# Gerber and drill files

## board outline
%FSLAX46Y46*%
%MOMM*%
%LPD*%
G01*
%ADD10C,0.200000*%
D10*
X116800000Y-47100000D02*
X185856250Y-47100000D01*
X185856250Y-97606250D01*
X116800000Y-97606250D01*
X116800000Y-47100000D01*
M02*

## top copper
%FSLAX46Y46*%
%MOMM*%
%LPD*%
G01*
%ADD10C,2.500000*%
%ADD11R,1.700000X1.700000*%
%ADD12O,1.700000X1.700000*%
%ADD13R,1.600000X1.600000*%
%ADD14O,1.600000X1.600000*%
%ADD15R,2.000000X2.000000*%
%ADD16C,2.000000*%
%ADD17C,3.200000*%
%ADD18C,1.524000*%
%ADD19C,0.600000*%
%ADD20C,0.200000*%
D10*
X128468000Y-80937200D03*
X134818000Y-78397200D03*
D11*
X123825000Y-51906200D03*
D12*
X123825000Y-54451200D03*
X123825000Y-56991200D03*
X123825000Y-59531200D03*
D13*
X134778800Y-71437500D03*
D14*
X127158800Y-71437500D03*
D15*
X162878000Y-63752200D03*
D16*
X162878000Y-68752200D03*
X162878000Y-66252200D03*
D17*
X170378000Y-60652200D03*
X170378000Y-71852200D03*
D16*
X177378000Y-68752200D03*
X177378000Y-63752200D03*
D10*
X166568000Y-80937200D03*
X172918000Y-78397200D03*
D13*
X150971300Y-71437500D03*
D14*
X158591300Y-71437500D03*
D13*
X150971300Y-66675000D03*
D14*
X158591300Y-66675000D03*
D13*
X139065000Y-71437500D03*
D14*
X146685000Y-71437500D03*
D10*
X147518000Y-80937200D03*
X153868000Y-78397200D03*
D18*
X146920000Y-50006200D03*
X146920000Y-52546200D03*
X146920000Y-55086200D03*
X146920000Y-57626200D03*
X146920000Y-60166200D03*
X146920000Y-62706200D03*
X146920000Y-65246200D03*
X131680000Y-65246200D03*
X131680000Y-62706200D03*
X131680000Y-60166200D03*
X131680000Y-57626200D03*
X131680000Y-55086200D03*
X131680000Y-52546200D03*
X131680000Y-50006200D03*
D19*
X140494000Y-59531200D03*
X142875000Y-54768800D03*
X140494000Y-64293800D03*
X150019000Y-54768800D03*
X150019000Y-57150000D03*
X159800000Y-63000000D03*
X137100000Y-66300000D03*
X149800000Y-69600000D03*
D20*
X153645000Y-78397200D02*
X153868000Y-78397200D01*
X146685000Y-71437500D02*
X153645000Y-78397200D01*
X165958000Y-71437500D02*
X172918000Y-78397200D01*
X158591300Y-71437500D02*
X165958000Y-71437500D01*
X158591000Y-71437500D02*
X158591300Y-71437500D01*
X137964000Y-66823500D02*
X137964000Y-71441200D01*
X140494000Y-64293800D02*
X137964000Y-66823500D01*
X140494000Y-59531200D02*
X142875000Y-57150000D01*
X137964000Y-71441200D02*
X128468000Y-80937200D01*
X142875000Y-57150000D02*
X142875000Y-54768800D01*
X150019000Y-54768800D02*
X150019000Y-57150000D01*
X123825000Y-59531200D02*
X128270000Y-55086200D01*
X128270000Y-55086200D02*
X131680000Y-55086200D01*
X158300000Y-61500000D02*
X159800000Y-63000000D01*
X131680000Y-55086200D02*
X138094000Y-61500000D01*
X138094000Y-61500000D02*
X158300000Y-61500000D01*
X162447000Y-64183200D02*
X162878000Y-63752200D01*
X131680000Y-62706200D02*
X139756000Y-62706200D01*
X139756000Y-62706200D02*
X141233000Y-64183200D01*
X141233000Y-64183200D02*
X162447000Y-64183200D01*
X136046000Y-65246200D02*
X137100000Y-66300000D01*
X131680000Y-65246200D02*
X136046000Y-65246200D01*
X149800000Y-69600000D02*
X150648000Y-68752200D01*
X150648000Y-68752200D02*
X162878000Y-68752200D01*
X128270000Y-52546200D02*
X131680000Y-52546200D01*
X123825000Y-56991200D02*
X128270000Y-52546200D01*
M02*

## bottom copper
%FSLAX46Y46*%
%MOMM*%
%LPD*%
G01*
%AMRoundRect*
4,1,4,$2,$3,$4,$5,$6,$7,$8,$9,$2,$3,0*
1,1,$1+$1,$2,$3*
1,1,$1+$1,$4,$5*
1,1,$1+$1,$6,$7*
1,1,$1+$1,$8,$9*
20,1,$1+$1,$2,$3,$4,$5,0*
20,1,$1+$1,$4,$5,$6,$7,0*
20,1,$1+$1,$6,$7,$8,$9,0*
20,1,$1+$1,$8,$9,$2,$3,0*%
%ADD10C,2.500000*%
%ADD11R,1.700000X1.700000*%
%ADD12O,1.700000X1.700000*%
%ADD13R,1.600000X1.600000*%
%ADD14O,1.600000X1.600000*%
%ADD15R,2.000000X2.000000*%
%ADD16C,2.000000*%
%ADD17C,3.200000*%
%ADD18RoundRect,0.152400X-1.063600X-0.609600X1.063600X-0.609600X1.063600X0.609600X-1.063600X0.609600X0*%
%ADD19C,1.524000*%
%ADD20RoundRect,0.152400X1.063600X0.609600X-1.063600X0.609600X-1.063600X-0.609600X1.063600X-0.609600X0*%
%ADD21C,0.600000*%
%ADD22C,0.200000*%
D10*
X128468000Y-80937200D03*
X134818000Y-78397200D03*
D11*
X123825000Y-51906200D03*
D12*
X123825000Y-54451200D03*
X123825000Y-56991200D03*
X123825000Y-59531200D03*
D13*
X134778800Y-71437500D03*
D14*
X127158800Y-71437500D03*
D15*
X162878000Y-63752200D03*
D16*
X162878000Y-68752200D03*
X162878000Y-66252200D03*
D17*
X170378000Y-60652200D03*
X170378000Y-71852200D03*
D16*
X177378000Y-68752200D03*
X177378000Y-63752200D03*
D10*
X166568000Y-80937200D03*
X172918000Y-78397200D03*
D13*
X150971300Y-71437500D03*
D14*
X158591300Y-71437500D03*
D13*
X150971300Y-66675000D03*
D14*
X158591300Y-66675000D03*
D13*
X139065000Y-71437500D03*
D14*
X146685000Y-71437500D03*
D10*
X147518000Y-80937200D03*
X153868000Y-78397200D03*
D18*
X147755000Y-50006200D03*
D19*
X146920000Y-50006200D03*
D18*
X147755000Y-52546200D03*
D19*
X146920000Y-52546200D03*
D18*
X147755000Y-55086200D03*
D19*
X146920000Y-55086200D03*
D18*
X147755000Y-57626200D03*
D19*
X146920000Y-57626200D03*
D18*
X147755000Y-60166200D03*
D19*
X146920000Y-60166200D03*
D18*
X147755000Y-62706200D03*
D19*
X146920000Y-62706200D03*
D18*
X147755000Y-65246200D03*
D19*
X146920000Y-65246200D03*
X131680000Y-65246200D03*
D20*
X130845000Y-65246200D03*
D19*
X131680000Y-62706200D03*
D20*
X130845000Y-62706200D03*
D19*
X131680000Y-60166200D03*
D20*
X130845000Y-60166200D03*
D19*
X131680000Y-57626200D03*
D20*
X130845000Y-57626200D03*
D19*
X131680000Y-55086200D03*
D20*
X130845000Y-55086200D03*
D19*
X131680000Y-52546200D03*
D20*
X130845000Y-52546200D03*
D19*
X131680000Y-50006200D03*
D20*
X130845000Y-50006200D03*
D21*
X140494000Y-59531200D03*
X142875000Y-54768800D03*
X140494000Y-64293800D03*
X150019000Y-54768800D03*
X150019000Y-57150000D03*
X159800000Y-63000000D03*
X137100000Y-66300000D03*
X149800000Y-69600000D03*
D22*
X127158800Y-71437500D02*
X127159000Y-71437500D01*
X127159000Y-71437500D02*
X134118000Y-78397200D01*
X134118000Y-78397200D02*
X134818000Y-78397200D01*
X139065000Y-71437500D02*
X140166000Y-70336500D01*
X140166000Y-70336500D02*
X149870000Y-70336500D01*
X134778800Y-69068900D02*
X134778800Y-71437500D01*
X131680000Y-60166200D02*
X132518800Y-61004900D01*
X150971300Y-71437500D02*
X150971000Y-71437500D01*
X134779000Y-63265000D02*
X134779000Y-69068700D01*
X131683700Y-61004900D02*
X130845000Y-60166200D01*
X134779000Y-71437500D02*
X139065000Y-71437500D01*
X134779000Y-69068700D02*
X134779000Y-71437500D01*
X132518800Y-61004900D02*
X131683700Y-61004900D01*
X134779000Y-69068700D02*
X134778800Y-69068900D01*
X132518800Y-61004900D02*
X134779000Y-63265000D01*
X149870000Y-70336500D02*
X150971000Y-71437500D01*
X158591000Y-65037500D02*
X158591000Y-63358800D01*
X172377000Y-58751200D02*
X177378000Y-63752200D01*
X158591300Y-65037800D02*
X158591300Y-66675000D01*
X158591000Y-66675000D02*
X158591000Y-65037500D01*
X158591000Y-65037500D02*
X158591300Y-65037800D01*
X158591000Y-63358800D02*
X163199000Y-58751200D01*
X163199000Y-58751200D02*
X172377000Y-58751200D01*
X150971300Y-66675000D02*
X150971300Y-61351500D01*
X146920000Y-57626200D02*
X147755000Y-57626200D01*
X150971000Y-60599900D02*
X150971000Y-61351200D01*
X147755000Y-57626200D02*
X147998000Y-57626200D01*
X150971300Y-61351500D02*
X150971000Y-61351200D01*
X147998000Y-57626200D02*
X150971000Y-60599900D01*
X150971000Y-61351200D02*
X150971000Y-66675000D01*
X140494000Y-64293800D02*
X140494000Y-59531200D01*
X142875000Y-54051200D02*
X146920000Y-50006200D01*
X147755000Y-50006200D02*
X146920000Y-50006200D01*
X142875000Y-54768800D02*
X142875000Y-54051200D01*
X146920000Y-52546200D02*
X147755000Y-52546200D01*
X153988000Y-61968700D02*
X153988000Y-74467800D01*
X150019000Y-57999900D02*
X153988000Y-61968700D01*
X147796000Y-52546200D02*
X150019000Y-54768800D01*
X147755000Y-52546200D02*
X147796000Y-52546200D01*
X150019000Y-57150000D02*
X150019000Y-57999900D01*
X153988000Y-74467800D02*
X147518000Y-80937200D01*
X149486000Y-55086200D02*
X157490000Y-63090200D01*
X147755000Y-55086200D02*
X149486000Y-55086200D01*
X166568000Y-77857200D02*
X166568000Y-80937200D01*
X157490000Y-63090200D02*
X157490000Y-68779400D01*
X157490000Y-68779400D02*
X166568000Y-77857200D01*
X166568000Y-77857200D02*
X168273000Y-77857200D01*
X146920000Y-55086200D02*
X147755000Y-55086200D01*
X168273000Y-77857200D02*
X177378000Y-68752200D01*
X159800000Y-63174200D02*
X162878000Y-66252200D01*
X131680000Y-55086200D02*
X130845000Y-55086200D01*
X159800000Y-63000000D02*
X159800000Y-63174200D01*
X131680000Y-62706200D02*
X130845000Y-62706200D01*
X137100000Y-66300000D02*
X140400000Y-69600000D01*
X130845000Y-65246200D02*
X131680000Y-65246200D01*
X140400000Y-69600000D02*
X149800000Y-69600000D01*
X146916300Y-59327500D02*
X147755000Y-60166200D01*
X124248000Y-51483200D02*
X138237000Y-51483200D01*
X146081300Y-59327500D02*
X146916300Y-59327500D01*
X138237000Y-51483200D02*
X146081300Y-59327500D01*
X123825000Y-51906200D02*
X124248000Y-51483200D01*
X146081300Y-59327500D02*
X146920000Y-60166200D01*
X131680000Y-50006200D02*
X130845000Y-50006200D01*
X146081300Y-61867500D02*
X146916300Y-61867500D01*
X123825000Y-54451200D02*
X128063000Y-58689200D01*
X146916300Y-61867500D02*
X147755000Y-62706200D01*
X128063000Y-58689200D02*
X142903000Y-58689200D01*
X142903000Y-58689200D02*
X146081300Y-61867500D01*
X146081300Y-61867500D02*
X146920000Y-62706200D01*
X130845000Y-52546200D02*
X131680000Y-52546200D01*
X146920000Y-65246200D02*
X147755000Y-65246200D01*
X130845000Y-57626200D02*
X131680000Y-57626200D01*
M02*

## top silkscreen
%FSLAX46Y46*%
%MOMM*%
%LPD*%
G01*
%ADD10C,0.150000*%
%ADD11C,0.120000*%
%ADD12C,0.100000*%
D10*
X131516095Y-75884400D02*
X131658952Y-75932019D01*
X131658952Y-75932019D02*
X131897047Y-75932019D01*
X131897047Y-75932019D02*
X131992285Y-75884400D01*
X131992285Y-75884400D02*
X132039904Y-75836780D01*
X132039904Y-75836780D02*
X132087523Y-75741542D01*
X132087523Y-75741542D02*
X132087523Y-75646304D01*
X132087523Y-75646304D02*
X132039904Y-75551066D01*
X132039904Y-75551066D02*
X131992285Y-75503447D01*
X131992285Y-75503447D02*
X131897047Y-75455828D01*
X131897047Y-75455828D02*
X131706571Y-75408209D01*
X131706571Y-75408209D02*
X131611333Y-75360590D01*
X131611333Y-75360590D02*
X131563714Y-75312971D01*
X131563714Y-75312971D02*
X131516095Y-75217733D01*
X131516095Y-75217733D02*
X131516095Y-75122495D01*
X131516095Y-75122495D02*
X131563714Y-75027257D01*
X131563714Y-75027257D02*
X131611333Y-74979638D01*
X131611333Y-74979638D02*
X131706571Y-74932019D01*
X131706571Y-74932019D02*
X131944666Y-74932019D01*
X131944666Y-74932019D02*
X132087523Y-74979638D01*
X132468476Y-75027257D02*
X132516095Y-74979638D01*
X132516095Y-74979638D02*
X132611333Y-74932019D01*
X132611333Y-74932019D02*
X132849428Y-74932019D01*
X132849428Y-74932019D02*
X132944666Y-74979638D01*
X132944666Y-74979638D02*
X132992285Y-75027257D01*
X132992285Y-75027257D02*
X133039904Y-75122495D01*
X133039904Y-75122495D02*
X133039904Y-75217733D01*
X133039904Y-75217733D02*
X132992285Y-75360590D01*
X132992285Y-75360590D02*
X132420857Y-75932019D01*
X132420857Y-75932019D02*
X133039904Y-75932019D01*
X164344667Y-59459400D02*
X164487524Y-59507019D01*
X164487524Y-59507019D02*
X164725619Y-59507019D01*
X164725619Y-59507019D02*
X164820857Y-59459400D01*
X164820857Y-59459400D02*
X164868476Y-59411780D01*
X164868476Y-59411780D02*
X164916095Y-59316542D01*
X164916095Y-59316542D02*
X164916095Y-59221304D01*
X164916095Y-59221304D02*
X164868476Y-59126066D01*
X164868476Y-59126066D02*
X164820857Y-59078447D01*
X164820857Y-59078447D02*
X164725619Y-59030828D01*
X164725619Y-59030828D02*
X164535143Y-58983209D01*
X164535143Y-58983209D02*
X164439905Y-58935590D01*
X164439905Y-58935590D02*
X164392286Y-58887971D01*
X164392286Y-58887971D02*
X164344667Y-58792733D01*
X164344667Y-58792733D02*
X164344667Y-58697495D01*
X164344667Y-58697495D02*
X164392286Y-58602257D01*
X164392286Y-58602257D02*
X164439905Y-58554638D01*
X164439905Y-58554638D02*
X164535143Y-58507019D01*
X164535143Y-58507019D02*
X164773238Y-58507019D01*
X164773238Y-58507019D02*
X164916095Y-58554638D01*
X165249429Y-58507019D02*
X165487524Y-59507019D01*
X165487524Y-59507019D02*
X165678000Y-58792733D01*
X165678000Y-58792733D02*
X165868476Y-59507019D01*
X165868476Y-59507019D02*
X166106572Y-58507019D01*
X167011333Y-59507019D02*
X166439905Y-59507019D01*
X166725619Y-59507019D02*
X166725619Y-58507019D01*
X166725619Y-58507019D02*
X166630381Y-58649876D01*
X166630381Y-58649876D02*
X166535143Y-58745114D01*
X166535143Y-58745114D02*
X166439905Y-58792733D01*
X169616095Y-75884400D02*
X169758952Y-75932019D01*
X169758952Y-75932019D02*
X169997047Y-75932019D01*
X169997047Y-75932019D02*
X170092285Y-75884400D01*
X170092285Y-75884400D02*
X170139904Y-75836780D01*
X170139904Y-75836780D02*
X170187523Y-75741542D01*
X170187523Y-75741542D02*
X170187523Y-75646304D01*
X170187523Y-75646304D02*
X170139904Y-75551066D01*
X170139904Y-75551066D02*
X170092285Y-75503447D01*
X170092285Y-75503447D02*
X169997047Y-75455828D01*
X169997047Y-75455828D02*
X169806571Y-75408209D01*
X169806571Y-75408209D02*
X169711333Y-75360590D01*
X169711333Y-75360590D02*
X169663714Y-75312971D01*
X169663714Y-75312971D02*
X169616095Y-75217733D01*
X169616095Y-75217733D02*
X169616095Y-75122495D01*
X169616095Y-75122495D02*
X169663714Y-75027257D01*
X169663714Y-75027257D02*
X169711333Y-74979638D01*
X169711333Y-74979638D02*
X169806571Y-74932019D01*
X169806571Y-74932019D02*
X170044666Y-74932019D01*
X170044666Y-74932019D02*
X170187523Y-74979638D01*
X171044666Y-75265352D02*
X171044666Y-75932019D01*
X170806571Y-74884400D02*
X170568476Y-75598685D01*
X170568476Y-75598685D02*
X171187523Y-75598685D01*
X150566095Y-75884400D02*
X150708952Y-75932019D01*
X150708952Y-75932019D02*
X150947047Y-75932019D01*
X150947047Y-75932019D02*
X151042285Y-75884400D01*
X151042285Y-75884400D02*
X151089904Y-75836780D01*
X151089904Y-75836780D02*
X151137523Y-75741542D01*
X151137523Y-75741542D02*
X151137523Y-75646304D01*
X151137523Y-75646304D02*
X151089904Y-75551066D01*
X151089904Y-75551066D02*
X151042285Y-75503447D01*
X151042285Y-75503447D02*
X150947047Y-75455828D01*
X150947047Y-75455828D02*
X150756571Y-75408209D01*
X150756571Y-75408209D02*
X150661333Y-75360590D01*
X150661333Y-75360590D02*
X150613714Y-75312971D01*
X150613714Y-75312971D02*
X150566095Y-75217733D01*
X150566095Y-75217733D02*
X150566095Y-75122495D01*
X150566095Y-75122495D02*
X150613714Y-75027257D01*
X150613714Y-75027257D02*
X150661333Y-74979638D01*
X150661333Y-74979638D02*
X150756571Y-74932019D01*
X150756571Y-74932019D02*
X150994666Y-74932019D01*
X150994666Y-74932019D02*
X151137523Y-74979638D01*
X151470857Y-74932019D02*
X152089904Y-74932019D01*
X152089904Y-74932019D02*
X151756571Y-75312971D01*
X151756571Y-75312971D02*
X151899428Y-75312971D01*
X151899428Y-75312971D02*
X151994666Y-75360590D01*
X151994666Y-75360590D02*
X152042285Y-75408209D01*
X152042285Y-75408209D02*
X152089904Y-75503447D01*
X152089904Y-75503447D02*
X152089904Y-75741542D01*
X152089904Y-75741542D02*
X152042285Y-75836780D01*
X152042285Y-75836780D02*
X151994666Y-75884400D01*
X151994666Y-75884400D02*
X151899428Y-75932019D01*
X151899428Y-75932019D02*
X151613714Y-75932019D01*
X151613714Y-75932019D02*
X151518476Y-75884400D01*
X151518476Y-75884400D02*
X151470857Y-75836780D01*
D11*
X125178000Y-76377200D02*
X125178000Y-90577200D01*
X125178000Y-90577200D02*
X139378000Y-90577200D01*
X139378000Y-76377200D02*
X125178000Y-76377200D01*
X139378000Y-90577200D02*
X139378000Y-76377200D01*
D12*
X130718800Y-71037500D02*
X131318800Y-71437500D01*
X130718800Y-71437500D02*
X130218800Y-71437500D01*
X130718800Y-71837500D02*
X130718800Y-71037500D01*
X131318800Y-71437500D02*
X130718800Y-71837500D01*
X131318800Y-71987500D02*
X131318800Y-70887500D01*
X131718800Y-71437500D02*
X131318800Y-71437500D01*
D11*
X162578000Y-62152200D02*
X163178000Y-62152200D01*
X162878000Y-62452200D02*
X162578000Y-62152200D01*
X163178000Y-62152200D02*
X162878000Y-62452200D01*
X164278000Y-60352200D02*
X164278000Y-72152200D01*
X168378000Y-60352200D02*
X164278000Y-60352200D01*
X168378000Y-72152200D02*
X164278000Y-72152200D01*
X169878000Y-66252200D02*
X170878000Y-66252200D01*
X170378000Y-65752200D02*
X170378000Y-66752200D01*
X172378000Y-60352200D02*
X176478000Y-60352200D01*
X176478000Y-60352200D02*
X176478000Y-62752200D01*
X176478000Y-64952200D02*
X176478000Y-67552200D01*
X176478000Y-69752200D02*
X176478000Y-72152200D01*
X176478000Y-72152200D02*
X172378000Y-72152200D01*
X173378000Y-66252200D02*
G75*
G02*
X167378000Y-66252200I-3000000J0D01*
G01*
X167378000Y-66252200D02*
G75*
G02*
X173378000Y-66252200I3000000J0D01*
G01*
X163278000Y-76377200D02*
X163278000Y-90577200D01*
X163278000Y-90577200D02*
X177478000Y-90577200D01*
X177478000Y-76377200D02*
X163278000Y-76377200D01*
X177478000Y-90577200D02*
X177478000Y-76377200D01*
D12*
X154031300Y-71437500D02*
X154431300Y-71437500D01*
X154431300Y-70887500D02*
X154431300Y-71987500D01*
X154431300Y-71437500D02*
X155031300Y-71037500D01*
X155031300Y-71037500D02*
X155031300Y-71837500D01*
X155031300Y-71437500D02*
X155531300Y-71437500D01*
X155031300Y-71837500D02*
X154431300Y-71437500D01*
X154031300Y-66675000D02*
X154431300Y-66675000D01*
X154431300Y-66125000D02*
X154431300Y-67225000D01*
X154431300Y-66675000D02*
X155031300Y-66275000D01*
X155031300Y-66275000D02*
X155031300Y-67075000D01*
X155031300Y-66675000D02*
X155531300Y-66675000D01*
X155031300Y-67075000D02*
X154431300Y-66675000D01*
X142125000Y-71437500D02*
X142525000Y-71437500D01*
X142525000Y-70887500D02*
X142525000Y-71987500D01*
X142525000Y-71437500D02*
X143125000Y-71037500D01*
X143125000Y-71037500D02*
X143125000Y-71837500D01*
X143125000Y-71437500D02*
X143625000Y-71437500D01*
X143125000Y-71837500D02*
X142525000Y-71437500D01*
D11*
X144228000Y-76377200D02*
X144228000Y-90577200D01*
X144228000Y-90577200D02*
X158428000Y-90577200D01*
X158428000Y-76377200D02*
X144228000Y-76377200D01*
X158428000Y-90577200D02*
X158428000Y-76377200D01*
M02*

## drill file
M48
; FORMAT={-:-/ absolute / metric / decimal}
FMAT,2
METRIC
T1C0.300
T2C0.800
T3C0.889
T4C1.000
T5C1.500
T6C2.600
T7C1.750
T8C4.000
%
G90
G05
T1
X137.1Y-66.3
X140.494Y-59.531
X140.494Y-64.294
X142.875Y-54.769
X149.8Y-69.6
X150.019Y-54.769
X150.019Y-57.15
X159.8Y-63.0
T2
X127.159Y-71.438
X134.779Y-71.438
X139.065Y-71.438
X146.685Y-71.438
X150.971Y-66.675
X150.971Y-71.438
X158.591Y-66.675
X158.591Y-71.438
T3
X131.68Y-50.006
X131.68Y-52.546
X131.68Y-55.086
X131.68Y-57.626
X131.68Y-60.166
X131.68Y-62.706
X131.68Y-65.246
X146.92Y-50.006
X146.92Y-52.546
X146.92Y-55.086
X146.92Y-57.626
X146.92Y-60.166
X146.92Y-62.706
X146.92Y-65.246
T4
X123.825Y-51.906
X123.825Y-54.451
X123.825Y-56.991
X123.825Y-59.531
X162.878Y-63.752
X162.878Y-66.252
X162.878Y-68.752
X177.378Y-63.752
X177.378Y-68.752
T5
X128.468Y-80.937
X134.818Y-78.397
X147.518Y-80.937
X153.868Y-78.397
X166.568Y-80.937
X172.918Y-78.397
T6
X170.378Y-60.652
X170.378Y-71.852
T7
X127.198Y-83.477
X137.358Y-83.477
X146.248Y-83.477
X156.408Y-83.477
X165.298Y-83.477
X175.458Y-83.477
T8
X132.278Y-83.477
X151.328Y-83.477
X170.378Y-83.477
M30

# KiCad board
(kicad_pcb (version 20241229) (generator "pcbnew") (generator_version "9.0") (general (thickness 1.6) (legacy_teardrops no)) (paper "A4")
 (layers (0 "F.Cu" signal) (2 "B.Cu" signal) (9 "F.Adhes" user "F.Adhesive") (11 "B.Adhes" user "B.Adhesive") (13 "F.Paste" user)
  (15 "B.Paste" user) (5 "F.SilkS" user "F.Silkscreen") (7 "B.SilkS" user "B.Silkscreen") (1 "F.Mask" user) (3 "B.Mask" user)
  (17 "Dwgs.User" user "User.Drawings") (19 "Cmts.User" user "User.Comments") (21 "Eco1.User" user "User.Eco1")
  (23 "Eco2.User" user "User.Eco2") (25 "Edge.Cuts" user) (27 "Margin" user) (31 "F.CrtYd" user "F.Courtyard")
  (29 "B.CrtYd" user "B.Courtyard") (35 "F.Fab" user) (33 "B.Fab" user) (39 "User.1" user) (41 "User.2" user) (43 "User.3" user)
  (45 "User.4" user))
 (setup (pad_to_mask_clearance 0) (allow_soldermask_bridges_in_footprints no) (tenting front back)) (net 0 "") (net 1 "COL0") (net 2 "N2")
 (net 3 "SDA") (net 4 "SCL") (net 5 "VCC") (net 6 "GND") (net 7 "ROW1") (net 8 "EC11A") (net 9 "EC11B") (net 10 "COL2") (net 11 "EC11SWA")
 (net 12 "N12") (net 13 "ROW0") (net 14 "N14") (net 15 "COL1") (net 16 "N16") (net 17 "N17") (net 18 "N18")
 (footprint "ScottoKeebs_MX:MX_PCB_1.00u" (layer "F.Cu") (at 132.278 83.4772)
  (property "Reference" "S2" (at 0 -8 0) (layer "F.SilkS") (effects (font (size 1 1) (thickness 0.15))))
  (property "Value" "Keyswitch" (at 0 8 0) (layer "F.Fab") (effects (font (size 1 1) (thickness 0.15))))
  (fp_line (start -7.1 -7.1) (end -7.1 7.1) (stroke (width 0.12) (type solid)) (layer "F.SilkS"))
  (fp_line (start -7.1 7.1) (end 7.1 7.1) (stroke (width 0.12) (type solid)) (layer "F.SilkS"))
  (fp_line (start 7.1 -7.1) (end -7.1 -7.1) (stroke (width 0.12) (type solid)) (layer "F.SilkS"))
  (fp_line (start 7.1 7.1) (end 7.1 -7.1) (stroke (width 0.12) (type solid)) (layer "F.SilkS"))
  (pad "" np_thru_hole circle (at -5.08 0) (size 1.75 1.75) (drill 1.75) (layers "*.Cu" "*.Mask"))
  (pad "" np_thru_hole circle (at 0 0) (size 4 4) (drill 4) (layers "*.Cu" "*.Mask"))
  (pad "" np_thru_hole circle (at 5.08 0) (size 1.75 1.75) (drill 1.75) (layers "*.Cu" "*.Mask"))
  (pad "1" thru_hole circle (at -3.81 -2.54) (size 2.5 2.5) (drill 1.5) (layers "*.Cu" "*.Mask") (remove_unused_layers no) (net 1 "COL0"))
  (pad "2" thru_hole circle (at 2.54 -5.08) (size 2.5 2.5) (drill 1.5) (layers "*.Cu" "*.Mask") (remove_unused_layers no) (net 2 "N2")))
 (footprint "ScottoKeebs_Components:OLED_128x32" (layer "F.Cu") (at 122.225 49.7312)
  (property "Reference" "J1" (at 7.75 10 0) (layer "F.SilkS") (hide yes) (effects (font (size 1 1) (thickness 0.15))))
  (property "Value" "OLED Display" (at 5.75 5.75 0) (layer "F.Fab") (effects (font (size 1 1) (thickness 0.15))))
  (pad "1" thru_hole rect (at 1.6 2.175 180) (size 1.7 1.7) (drill 1) (layers "*.Cu" "*.Mask") (remove_unused_layers no) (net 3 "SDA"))
  (pad "2" thru_hole oval (at 1.6 4.72 180) (size 1.7 1.7) (drill 1) (layers "*.Cu" "*.Mask") (remove_unused_layers no) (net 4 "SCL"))
  (pad "3" thru_hole oval (at 1.6 7.26 180) (size 1.7 1.7) (drill 1) (layers "*.Cu" "*.Mask") (remove_unused_layers no) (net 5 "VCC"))
  (pad "4" thru_hole oval (at 1.6 9.8 180) (size 1.7 1.7) (drill 1) (layers "*.Cu" "*.Mask") (remove_unused_layers no) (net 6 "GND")))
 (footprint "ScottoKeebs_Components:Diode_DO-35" (layer "F.Cu") (at 134.7788 71.4375 180)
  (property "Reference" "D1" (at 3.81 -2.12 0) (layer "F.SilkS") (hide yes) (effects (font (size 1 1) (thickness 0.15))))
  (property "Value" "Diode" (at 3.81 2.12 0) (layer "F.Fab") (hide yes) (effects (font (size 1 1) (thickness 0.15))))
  (fp_line (start 4.06 0.4) (end 3.46 0) (stroke (width 0.1) (type solid)) (layer "F.SilkS"))
  (fp_line (start 4.06 0) (end 4.56 0) (stroke (width 0.1) (type solid)) (layer "F.SilkS"))
  (fp_line (start 4.06 -0.4) (end 4.06 0.4) (stroke (width 0.1) (type solid)) (layer "F.SilkS"))
  (fp_line (start 3.46 0) (end 4.06 -0.4) (stroke (width 0.1) (type solid)) (layer "F.SilkS"))
  (fp_line (start 3.46 -0.55) (end 3.46 0.55) (stroke (width 0.1) (type solid)) (layer "F.SilkS"))
  (fp_line (start 3.06 0) (end 3.46 0) (stroke (width 0.1) (type solid)) (layer "F.SilkS"))
  (pad "1" thru_hole rect (at 0 0 180) (size 1.6 1.6) (drill 0.8) (layers "*.Cu" "*.Mask") (remove_unused_layers no) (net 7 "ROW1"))
  (pad "2" thru_hole oval (at 7.62 0 180) (size 1.6 1.6) (drill 0.8) (layers "*.Cu" "*.Mask") (remove_unused_layers no) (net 2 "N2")))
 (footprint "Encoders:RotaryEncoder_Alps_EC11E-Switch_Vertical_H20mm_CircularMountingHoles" (layer "F.Cu") (at 162.878 63.7522)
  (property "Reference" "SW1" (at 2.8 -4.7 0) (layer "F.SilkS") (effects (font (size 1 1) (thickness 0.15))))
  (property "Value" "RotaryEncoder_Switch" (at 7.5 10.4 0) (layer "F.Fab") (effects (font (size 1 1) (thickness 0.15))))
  (fp_line (start -0.3 -1.6) (end 0.3 -1.6) (stroke (width 0.12) (type solid)) (layer "F.SilkS"))
  (fp_line (start 0 -1.3) (end -0.3 -1.6) (stroke (width 0.12) (type solid)) (layer "F.SilkS"))
  (fp_line (start 0.3 -1.6) (end 0 -1.3) (stroke (width 0.12) (type solid)) (layer "F.SilkS"))
  (fp_line (start 1.4 -3.4) (end 1.4 8.4) (stroke (width 0.12) (type solid)) (layer "F.SilkS"))
  (fp_line (start 5.5 -3.4) (end 1.4 -3.4) (stroke (width 0.12) (type solid)) (layer "F.SilkS"))
  (fp_line (start 5.5 8.4) (end 1.4 8.4) (stroke (width 0.12) (type solid)) (layer "F.SilkS"))
  (fp_line (start 7 2.5) (end 8 2.5) (stroke (width 0.12) (type solid)) (layer "F.SilkS"))
  (fp_line (start 7.5 2) (end 7.5 3) (stroke (width 0.12) (type solid)) (layer "F.SilkS"))
  (fp_line (start 9.5 -3.4) (end 13.6 -3.4) (stroke (width 0.12) (type solid)) (layer "F.SilkS"))
  (fp_line (start 13.6 -3.4) (end 13.6 -1) (stroke (width 0.12) (type solid)) (layer "F.SilkS"))
  (fp_line (start 13.6 1.2) (end 13.6 3.8) (stroke (width 0.12) (type solid)) (layer "F.SilkS"))
  (fp_line (start 13.6 6) (end 13.6 8.4) (stroke (width 0.12) (type solid)) (layer "F.SilkS"))
  (fp_line (start 13.6 8.4) (end 9.5 8.4) (stroke (width 0.12) (type solid)) (layer "F.SilkS"))
  (fp_circle (center 7.5 2.5) (end 10.5 2.5) (stroke (width 0.12) (type solid)) (fill no) (layer "F.SilkS"))
  (pad "A" thru_hole rect (at 0 0) (size 2 2) (drill 1) (layers "*.Cu" "*.Mask") (remove_unused_layers no) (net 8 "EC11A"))
  (pad "B" thru_hole circle (at 0 5) (size 2 2) (drill 1) (layers "*.Cu" "*.Mask") (remove_unused_layers no) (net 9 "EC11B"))
  (pad "C" thru_hole circle (at 0 2.5) (size 2 2) (drill 1) (layers "*.Cu" "*.Mask") (remove_unused_layers no) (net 6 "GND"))
  (pad "MP" thru_hole circle (at 7.5 -3.1) (size 3.2 3.2) (drill 2.6) (layers "*.Cu" "*.Mask") (remove_unused_layers no))
  (pad "MP" thru_hole circle (at 7.5 8.1) (size 3.2 3.2) (drill 2.6) (layers "*.Cu" "*.Mask") (remove_unused_layers no))
  (pad "S1" thru_hole circle (at 14.5 5) (size 2 2) (drill 1) (layers "*.Cu" "*.Mask") (remove_unused_layers no) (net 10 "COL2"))
  (pad "S2" thru_hole circle (at 14.5 0) (size 2 2) (drill 1) (layers "*.Cu" "*.Mask") (remove_unused_layers no) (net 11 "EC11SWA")))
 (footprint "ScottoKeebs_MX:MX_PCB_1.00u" (layer "F.Cu") (at 170.378 83.4772)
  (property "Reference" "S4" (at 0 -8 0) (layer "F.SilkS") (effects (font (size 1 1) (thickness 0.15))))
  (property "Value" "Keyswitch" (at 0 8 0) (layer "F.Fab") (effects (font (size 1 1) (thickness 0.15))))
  (fp_line (start -7.1 -7.1) (end -7.1 7.1) (stroke (width 0.12) (type solid)) (layer "F.SilkS"))
  (fp_line (start -7.1 7.1) (end 7.1 7.1) (stroke (width 0.12) (type solid)) (layer "F.SilkS"))
  (fp_line (start 7.1 -7.1) (end -7.1 -7.1) (stroke (width 0.12) (type solid)) (layer "F.SilkS"))
  (fp_line (start 7.1 7.1) (end 7.1 -7.1) (stroke (width 0.12) (type solid)) (layer "F.SilkS"))
  (pad "" np_thru_hole circle (at -5.08 0) (size 1.75 1.75) (drill 1.75) (layers "*.Cu" "*.Mask"))
  (pad "" np_thru_hole circle (at 0 0) (size 4 4) (drill 4) (layers "*.Cu" "*.Mask"))
  (pad "" np_thru_hole circle (at 5.08 0) (size 1.75 1.75) (drill 1.75) (layers "*.Cu" "*.Mask"))
  (pad "1" thru_hole circle (at -3.81 -2.54) (size 2.5 2.5) (drill 1.5) (layers "*.Cu" "*.Mask") (remove_unused_layers no) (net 10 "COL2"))
  (pad "2" thru_hole circle (at 2.54 -5.08) (size 2.5 2.5) (drill 1.5) (layers "*.Cu" "*.Mask") (remove_unused_layers no) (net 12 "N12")))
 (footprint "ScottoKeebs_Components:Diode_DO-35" (layer "F.Cu") (at 150.9713 71.4375)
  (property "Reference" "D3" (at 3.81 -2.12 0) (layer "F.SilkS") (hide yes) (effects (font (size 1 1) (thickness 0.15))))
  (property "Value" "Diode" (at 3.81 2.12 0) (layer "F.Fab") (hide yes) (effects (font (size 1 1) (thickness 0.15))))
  (fp_line (start 3.06 0) (end 3.46 0) (stroke (width 0.1) (type solid)) (layer "F.SilkS"))
  (fp_line (start 3.46 -0.55) (end 3.46 0.55) (stroke (width 0.1) (type solid)) (layer "F.SilkS"))
  (fp_line (start 3.46 0) (end 4.06 -0.4) (stroke (width 0.1) (type solid)) (layer "F.SilkS"))
  (fp_line (start 4.06 -0.4) (end 4.06 0.4) (stroke (width 0.1) (type solid)) (layer "F.SilkS"))
  (fp_line (start 4.06 0) (end 4.56 0) (stroke (width 0.1) (type solid)) (layer "F.SilkS"))
  (fp_line (start 4.06 0.4) (end 3.46 0) (stroke (width 0.1) (type solid)) (layer "F.SilkS"))
  (pad "1" thru_hole rect (at 0 0) (size 1.6 1.6) (drill 0.8) (layers "*.Cu" "*.Mask") (remove_unused_layers no) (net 7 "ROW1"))
  (pad "2" thru_hole oval (at 7.62 0) (size 1.6 1.6) (drill 0.8) (layers "*.Cu" "*.Mask") (remove_unused_layers no) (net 12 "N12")))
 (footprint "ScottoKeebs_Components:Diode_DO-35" (layer "F.Cu") (at 150.9713 66.675)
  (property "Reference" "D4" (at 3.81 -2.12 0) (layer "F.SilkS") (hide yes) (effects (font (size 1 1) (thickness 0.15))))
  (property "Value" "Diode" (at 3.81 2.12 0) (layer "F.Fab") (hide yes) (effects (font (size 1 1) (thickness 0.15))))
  (fp_line (start 3.06 0) (end 3.46 0) (stroke (width 0.1) (type solid)) (layer "F.SilkS"))
  (fp_line (start 3.46 -0.55) (end 3.46 0.55) (stroke (width 0.1) (type solid)) (layer "F.SilkS"))
  (fp_line (start 3.46 0) (end 4.06 -0.4) (stroke (width 0.1) (type solid)) (layer "F.SilkS"))
  (fp_line (start 4.06 -0.4) (end 4.06 0.4) (stroke (width 0.1) (type solid)) (layer "F.SilkS"))
  (fp_line (start 4.06 0) (end 4.56 0) (stroke (width 0.1) (type solid)) (layer "F.SilkS"))
  (fp_line (start 4.06 0.4) (end 3.46 0) (stroke (width 0.1) (type solid)) (layer "F.SilkS"))
  (pad "1" thru_hole rect (at 0 0) (size 1.6 1.6) (drill 0.8) (layers "*.Cu" "*.Mask") (remove_unused_layers no) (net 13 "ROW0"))
  (pad "2" thru_hole oval (at 7.62 0) (size 1.6 1.6) (drill 0.8) (layers "*.Cu" "*.Mask") (remove_unused_layers no) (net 11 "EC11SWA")))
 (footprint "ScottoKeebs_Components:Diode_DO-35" (layer "F.Cu") (at 139.065 71.4375)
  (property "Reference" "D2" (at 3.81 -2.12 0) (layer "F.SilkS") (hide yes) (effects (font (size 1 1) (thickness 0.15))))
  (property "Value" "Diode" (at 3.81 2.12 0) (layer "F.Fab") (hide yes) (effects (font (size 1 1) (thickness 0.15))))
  (fp_line (start 3.06 0) (end 3.46 0) (stroke (width 0.1) (type solid)) (layer "F.SilkS"))
  (fp_line (start 3.46 -0.55) (end 3.46 0.55) (stroke (width 0.1) (type solid)) (layer "F.SilkS"))
  (fp_line (start 3.46 0) (end 4.06 -0.4) (stroke (width 0.1) (type solid)) (layer "F.SilkS"))
  (fp_line (start 4.06 -0.4) (end 4.06 0.4) (stroke (width 0.1) (type solid)) (layer "F.SilkS"))
  (fp_line (start 4.06 0) (end 4.56 0) (stroke (width 0.1) (type solid)) (layer "F.SilkS"))
  (fp_line (start 4.06 0.4) (end 3.46 0) (stroke (width 0.1) (type solid)) (layer "F.SilkS"))
  (pad "1" thru_hole rect (at 0 0) (size 1.6 1.6) (drill 0.8) (layers "*.Cu" "*.Mask") (remove_unused_layers no) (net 7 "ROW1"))
  (pad "2" thru_hole oval (at 7.62 0) (size 1.6 1.6) (drill 0.8) (layers "*.Cu" "*.Mask") (remove_unused_layers no) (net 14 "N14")))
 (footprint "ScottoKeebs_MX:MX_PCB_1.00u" (layer "F.Cu") (at 151.328 83.4772)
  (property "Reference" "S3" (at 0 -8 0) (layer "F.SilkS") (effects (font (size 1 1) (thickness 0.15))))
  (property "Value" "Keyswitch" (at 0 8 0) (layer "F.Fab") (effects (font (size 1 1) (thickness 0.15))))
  (fp_line (start -7.1 -7.1) (end -7.1 7.1) (stroke (width 0.12) (type solid)) (layer "F.SilkS"))
  (fp_line (start -7.1 7.1) (end 7.1 7.1) (stroke (width 0.12) (type solid)) (layer "F.SilkS"))
  (fp_line (start 7.1 -7.1) (end -7.1 -7.1) (stroke (width 0.12) (type solid)) (layer "F.SilkS"))
  (fp_line (start 7.1 7.1) (end 7.1 -7.1) (stroke (width 0.12) (type solid)) (layer "F.SilkS"))
  (pad "" np_thru_hole circle (at -5.08 0) (size 1.75 1.75) (drill 1.75) (layers "*.Cu" "*.Mask"))
  (pad "" np_thru_hole circle (at 0 0) (size 4 4) (drill 4) (layers "*.Cu" "*.Mask"))
  (pad "" np_thru_hole circle (at 5.08 0) (size 1.75 1.75) (drill 1.75) (layers "*.Cu" "*.Mask"))
  (pad "1" thru_hole circle (at -3.81 -2.54) (size 2.5 2.5) (drill 1.5) (layers "*.Cu" "*.Mask") (remove_unused_layers no) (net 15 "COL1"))
  (pad "2" thru_hole circle (at 2.54 -5.08) (size 2.5 2.5) (drill 1.5) (layers "*.Cu" "*.Mask") (remove_unused_layers no) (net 14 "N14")))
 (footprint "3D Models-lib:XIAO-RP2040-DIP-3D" (layer "B.Cu") (at 139.3 57.6262 180)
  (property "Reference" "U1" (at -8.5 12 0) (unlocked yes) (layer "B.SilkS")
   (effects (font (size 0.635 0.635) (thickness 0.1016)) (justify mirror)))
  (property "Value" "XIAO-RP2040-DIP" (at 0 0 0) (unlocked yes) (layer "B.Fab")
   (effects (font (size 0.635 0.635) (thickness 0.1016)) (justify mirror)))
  (pad "1" smd roundrect (at -8.455 7.62) (size 2.432 1.524) (layers "B.Cu" "B.Mask") (roundrect_rratio 0.1) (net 1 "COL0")
   (thermal_bridge_angle 45))
  (pad "1" thru_hole circle (at -7.62 7.62) (size 1.524 1.524) (drill 0.889) (layers "*.Cu" "*.Mask") (remove_unused_layers no)
   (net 1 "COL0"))
  (pad "2" smd roundrect (at -8.455 5.08) (size 2.432 1.524) (layers "B.Cu" "B.Mask") (roundrect_rratio 0.1) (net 15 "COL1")
   (thermal_bridge_angle 45))
  (pad "2" thru_hole circle (at -7.62 5.08) (size 1.524 1.524) (drill 0.889) (layers "*.Cu" "*.Mask") (remove_unused_layers no)
   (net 15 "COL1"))
  (pad "3" smd roundrect (at -8.455 2.54) (size 2.432 1.524) (layers "B.Cu" "B.Mask") (roundrect_rratio 0.1) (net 10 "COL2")
   (thermal_bridge_angle 45))
  (pad "3" thru_hole circle (at -7.62 2.54) (size 1.524 1.524) (drill 0.889) (layers "*.Cu" "*.Mask") (remove_unused_layers no)
   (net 10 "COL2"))
  (pad "4" smd roundrect (at -8.455 0) (size 2.432 1.524) (layers "B.Cu" "B.Mask") (roundrect_rratio 0.1) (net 13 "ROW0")
   (thermal_bridge_angle 45))
  (pad "4" thru_hole circle (at -7.62 0) (size 1.524 1.524) (drill 0.889) (layers "*.Cu" "*.Mask") (remove_unused_layers no) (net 13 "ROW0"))
  (pad "5" smd roundrect (at -8.455 -2.54) (size 2.432 1.524) (layers "B.Cu" "B.Mask") (roundrect_rratio 0.1) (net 3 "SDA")
   (thermal_bridge_angle 45))
  (pad "5" thru_hole circle (at -7.62 -2.54) (size 1.524 1.524) (drill 0.889) (layers "*.Cu" "*.Mask") (remove_unused_layers no)
   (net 3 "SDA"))
  (pad "6" smd roundrect (at -8.455 -5.08) (size 2.432 1.524) (layers "B.Cu" "B.Mask") (roundrect_rratio 0.1) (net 4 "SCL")
   (thermal_bridge_angle 45))
  (pad "6" thru_hole circle (at -7.62 -5.08) (size 1.524 1.524) (drill 0.889) (layers "*.Cu" "*.Mask") (remove_unused_layers no)
   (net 4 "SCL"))
  (pad "7" smd roundrect (at -8.455 -7.62) (size 2.432 1.524) (layers "B.Cu" "B.Mask") (roundrect_rratio 0.1) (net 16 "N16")
   (thermal_bridge_angle 45))
  (pad "7" thru_hole circle (at -7.62 -7.62) (size 1.524 1.524) (drill 0.889) (layers "*.Cu" "*.Mask") (remove_unused_layers no)
   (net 16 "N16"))
  (pad "8" thru_hole circle (at 7.62 -7.62 180) (size 1.524 1.524) (drill 0.889) (layers "*.Cu" "*.Mask") (remove_unused_layers no)
   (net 9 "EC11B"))
  (pad "8" smd roundrect (at 8.455 -7.62 180) (size 2.432 1.524) (layers "B.Cu" "B.Mask") (roundrect_rratio 0.1) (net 9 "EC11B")
   (thermal_bridge_angle 45))
  (pad "9" thru_hole circle (at 7.62 -5.08 180) (size 1.524 1.524) (drill 0.889) (layers "*.Cu" "*.Mask") (remove_unused_layers no)
   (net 8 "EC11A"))
  (pad "9" smd roundrect (at 8.455 -5.08 180) (size 2.432 1.524) (layers "B.Cu" "B.Mask") (roundrect_rratio 0.1) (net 8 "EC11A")
   (thermal_bridge_angle 45))
  (pad "10" thru_hole circle (at 7.62 -2.54 180) (size 1.524 1.524) (drill 0.889) (layers "*.Cu" "*.Mask") (remove_unused_layers no)
   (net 7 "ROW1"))
  (pad "10" smd roundrect (at 8.455 -2.54 180) (size 2.432 1.524) (layers "B.Cu" "B.Mask") (roundrect_rratio 0.1) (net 7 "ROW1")
   (thermal_bridge_angle 45))
  (pad "11" thru_hole circle (at 7.62 0 180) (size 1.524 1.524) (drill 0.889) (layers "*.Cu" "*.Mask") (remove_unused_layers no)
   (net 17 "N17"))
  (pad "11" smd roundrect (at 8.455 0 180) (size 2.432 1.524) (layers "B.Cu" "B.Mask") (roundrect_rratio 0.1) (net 17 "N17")
   (thermal_bridge_angle 45))
  (pad "12" thru_hole circle (at 7.62 2.54 180) (size 1.524 1.524) (drill 0.889) (layers "*.Cu" "*.Mask") (remove_unused_layers no)
   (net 6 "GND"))
  (pad "12" smd roundrect (at 8.455 2.54 180) (size 2.432 1.524) (layers "B.Cu" "B.Mask") (roundrect_rratio 0.1) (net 6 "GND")
   (thermal_bridge_angle 45))
  (pad "13" thru_hole circle (at 7.62 5.08 180) (size 1.524 1.524) (drill 0.889) (layers "*.Cu" "*.Mask") (remove_unused_layers no)
   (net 5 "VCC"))
  (pad "13" smd roundrect (at 8.455 5.08 180) (size 2.432 1.524) (layers "B.Cu" "B.Mask") (roundrect_rratio 0.1) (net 5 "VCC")
   (thermal_bridge_angle 45))
  (pad "14" thru_hole circle (at 7.62 7.62 180) (size 1.524 1.524) (drill 0.889) (layers "*.Cu" "*.Mask") (remove_unused_layers no)
   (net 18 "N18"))
  (pad "14" smd roundrect (at 8.455 7.62 180) (size 2.432 1.524) (layers "B.Cu" "B.Mask") (roundrect_rratio 0.1) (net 18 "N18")
   (thermal_bridge_angle 45)))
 (gr_rect (start 116.8 47.1) (end 185.85625 97.60625) (stroke (width 0.2) (type solid)) (fill no) (layer "Edge.Cuts"))
 (segment (start 127.1588 71.4375) (end 127.159 71.4375) (width 0.2) (layer "B.Cu") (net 2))
 (segment (start 127.159 71.4375) (end 134.118 78.3972) (width 0.2) (layer "B.Cu") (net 2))
 (segment (start 134.118 78.3972) (end 134.818 78.3972) (width 0.2) (layer "B.Cu") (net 2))
 (segment (start 139.065 71.4375) (end 140.166 70.3365) (width 0.2) (layer "B.Cu") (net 7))
 (segment (start 140.166 70.3365) (end 149.87 70.3365) (width 0.2) (layer "B.Cu") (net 7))
 (segment (start 134.7788 69.0689) (end 134.7788 71.4375) (width 0.2) (layer "B.Cu") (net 7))
 (segment (start 131.68 60.1662) (end 132.5188 61.0049) (width 0.2) (layer "B.Cu") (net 7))
 (segment (start 150.9713 71.4375) (end 150.971 71.4375) (width 0.2) (layer "B.Cu") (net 7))
 (segment (start 134.779 63.265) (end 134.779 69.0687) (width 0.2) (layer "B.Cu") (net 7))
 (segment (start 131.6837 61.0049) (end 130.845 60.1662) (width 0.2) (layer "B.Cu") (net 7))
 (segment (start 134.779 71.4375) (end 139.065 71.4375) (width 0.2) (layer "B.Cu") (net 7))
 (segment (start 134.779 69.0687) (end 134.779 71.4375) (width 0.2) (layer "B.Cu") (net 7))
 (segment (start 132.5188 61.0049) (end 131.6837 61.0049) (width 0.2) (layer "B.Cu") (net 7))
 (segment (start 134.779 69.0687) (end 134.7788 69.0689) (width 0.2) (layer "B.Cu") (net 7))
 (segment (start 132.5188 61.0049) (end 134.779 63.265) (width 0.2) (layer "B.Cu") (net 7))
 (segment (start 149.87 70.3365) (end 150.971 71.4375) (width 0.2) (layer "B.Cu") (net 7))
 (segment (start 153.645 78.3972) (end 153.868 78.3972) (width 0.2) (layer "F.Cu") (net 14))
 (segment (start 146.685 71.4375) (end 153.645 78.3972) (width 0.2) (layer "F.Cu") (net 14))
 (segment (start 165.958 71.4375) (end 172.918 78.3972) (width 0.2) (layer "F.Cu") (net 12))
 (segment (start 158.5913 71.4375) (end 165.958 71.4375) (width 0.2) (layer "F.Cu") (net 12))
 (segment (start 158.591 71.4375) (end 158.5913 71.4375) (width 0.2) (layer "F.Cu") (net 12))
 (segment (start 158.591 65.0375) (end 158.591 63.3588) (width 0.2) (layer "B.Cu") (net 11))
 (segment (start 172.377 58.7512) (end 177.378 63.7522) (width 0.2) (layer "B.Cu") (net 11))
 (segment (start 158.5913 65.0378) (end 158.5913 66.675) (width 0.2) (layer "B.Cu") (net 11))
 (segment (start 158.591 66.675) (end 158.591 65.0375) (width 0.2) (layer "B.Cu") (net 11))
 (segment (start 158.591 65.0375) (end 158.5913 65.0378) (width 0.2) (layer "B.Cu") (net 11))
 (segment (start 158.591 63.3588) (end 163.199 58.7512) (width 0.2) (layer "B.Cu") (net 11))
 (segment (start 163.199 58.7512) (end 172.377 58.7512) (width 0.2) (layer "B.Cu") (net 11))
 (segment (start 150.9713 66.675) (end 150.9713 61.3515) (width 0.2) (layer "B.Cu") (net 13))
 (segment (start 146.92 57.6262) (end 147.755 57.6262) (width 0.2) (layer "B.Cu") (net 13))
 (segment (start 150.971 60.5999) (end 150.971 61.3512) (width 0.2) (layer "B.Cu") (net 13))
 (segment (start 147.755 57.6262) (end 147.998 57.6262) (width 0.2) (layer "B.Cu") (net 13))
 (segment (start 150.9713 61.3515) (end 150.971 61.3512) (width 0.2) (layer "B.Cu") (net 13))
 (segment (start 147.998 57.6262) (end 150.971 60.5999) (width 0.2) (layer "B.Cu") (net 13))
 (segment (start 150.971 61.3512) (end 150.971 66.675) (width 0.2) (layer "B.Cu") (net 13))
 (segment (start 137.964 66.8235) (end 137.964 71.4412) (width 0.2) (layer "F.Cu") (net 1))
 (segment (start 140.494 64.2938) (end 137.964 66.8235) (width 0.2) (layer "F.Cu") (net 1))
 (segment (start 140.494 59.5312) (end 142.875 57.15) (width 0.2) (layer "F.Cu") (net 1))
 (segment (start 137.964 71.4412) (end 128.468 80.9372) (width 0.2) (layer "F.Cu") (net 1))
 (segment (start 142.875 57.15) (end 142.875 54.7688) (width 0.2) (layer "F.Cu") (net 1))
 (via (at 140.494 59.5312) (size 0.6) (drill 0.3) (layers "F.Cu" "B.Cu") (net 1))
 (via (at 142.875 54.7688) (size 0.6) (drill 0.3) (layers "F.Cu" "B.Cu") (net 1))
 (via (at 140.494 64.2938) (size 0.6) (drill 0.3) (layers "F.Cu" "B.Cu") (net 1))
 (segment (start 140.494 64.2938) (end 140.494 59.5312) (width 0.2) (layer "B.Cu") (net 1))
 (segment (start 142.875 54.0512) (end 146.92 50.0062) (width 0.2) (layer "B.Cu") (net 1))
 (segment (start 147.755 50.0062) (end 146.92 50.0062) (width 0.2) (layer "B.Cu") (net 1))
 (segment (start 142.875 54.7688) (end 142.875 54.0512) (width 0.2) (layer "B.Cu") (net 1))
 (segment (start 150.019 54.7688) (end 150.019 57.15) (width 0.2) (layer "F.Cu") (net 15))
 (via (at 150.019 54.7688) (size 0.6) (drill 0.3) (layers "F.Cu" "B.Cu") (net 15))
 (via (at 150.019 57.15) (size 0.6) (drill 0.3) (layers "F.Cu" "B.Cu") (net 15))
 (segment (start 146.92 52.5462) (end 147.755 52.5462) (width 0.2) (layer "B.Cu") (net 15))
 (segment (start 153.988 61.9687) (end 153.988 74.4678) (width 0.2) (layer "B.Cu") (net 15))
 (segment (start 150.019 57.9999) (end 153.988 61.9687) (width 0.2) (layer "B.Cu") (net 15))
 (segment (start 147.796 52.5462) (end 150.019 54.7688) (width 0.2) (layer "B.Cu") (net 15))
 (segment (start 147.755 52.5462) (end 147.796 52.5462) (width 0.2) (layer "B.Cu") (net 15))
 (segment (start 150.019 57.15) (end 150.019 57.9999) (width 0.2) (layer "B.Cu") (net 15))
 (segment (start 153.988 74.4678) (end 147.518 80.9372) (width 0.2) (layer "B.Cu") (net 15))
 (segment (start 149.486 55.0862) (end 157.49 63.0902) (width 0.2) (layer "B.Cu") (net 10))
 (segment (start 147.755 55.0862) (end 149.486 55.0862) (width 0.2) (layer "B.Cu") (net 10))
 (segment (start 166.568 77.8572) (end 166.568 80.9372) (width 0.2) (layer "B.Cu") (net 10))
 (segment (start 157.49 63.0902) (end 157.49 68.7794) (width 0.2) (layer "B.Cu") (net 10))
 (segment (start 157.49 68.7794) (end 166.568 77.8572) (width 0.2) (layer "B.Cu") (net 10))
 (segment (start 166.568 77.8572) (end 168.273 77.8572) (width 0.2) (layer "B.Cu") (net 10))
 (segment (start 146.92 55.0862) (end 147.755 55.0862) (width 0.2) (layer "B.Cu") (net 10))
 (segment (start 168.273 77.8572) (end 177.378 68.7522) (width 0.2) (layer "B.Cu") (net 10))
 (segment (start 123.825 59.5312) (end 128.27 55.0862) (width 0.2) (layer "F.Cu") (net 6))
 (segment (start 128.27 55.0862) (end 131.68 55.0862) (width 0.2) (layer "F.Cu") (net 6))
 (segment (start 158.3 61.5) (end 159.8 63) (width 0.2) (layer "F.Cu") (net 6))
 (segment (start 131.68 55.0862) (end 138.094 61.5) (width 0.2) (layer "F.Cu") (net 6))
 (segment (start 138.094 61.5) (end 158.3 61.5) (width 0.2) (layer "F.Cu") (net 6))
 (via (at 159.8 63) (size 0.6) (drill 0.3) (layers "F.Cu" "B.Cu") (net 6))
 (segment (start 159.8 63.1742) (end 162.878 66.2522) (width 0.2) (layer "B.Cu") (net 6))
 (segment (start 131.68 55.0862) (end 130.845 55.0862) (width 0.2) (layer "B.Cu") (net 6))
 (segment (start 159.8 63) (end 159.8 63.1742) (width 0.2) (layer "B.Cu") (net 6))
 (segment (start 162.447 64.1832) (end 162.878 63.7522) (width 0.2) (layer "F.Cu") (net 8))
 (segment (start 131.68 62.7062) (end 139.756 62.7062) (width 0.2) (layer "F.Cu") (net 8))
 (segment (start 139.756 62.7062) (end 141.233 64.1832) (width 0.2) (layer "F.Cu") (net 8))
 (segment (start 141.233 64.1832) (end 162.447 64.1832) (width 0.2) (layer "F.Cu") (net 8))
 (segment (start 131.68 62.7062) (end 130.845 62.7062) (width 0.2) (layer "B.Cu") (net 8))
 (segment (start 136.046 65.2462) (end 137.1 66.3) (width 0.2) (layer "F.Cu") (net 9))
 (segment (start 131.68 65.2462) (end 136.046 65.2462) (width 0.2) (layer "F.Cu") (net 9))
 (segment (start 149.8 69.6) (end 150.648 68.7522) (width 0.2) (layer "F.Cu") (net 9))
 (segment (start 150.648 68.7522) (end 162.878 68.7522) (width 0.2) (layer "F.Cu") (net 9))
 (via (at 137.1 66.3) (size 0.6) (drill 0.3) (layers "F.Cu" "B.Cu") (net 9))
 (via (at 149.8 69.6) (size 0.6) (drill 0.3) (layers "F.Cu" "B.Cu") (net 9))
 (segment (start 137.1 66.3) (end 140.4 69.6) (width 0.2) (layer "B.Cu") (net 9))
 (segment (start 130.845 65.2462) (end 131.68 65.2462) (width 0.2) (layer "B.Cu") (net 9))
 (segment (start 140.4 69.6) (end 149.8 69.6) (width 0.2) (layer "B.Cu") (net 9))
 (segment (start 146.9163 59.3275) (end 147.755 60.1662) (width 0.2) (layer "B.Cu") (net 3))
 (segment (start 124.248 51.4832) (end 138.237 51.4832) (width 0.2) (layer "B.Cu") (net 3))
 (segment (start 146.0813 59.3275) (end 146.9163 59.3275) (width 0.2) (layer "B.Cu") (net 3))
 (segment (start 138.237 51.4832) (end 146.0813 59.3275) (width 0.2) (layer "B.Cu") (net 3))
 (segment (start 123.825 51.9062) (end 124.248 51.4832) (width 0.2) (layer "B.Cu") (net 3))
 (segment (start 146.0813 59.3275) (end 146.92 60.1662) (width 0.2) (layer "B.Cu") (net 3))
 (segment (start 131.68 50.0062) (end 130.845 50.0062) (width 0.2) (layer "B.Cu") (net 18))
 (segment (start 146.0813 61.8675) (end 146.9163 61.8675) (width 0.2) (layer "B.Cu") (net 4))
 (segment (start 123.825 54.4512) (end 128.063 58.6892) (width 0.2) (layer "B.Cu") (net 4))
 (segment (start 146.9163 61.8675) (end 147.755 62.7062) (width 0.2) (layer "B.Cu") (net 4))
 (segment (start 128.063 58.6892) (end 142.903 58.6892) (width 0.2) (layer "B.Cu") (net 4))
 (segment (start 142.903 58.6892) (end 146.0813 61.8675) (width 0.2) (layer "B.Cu") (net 4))
 (segment (start 146.0813 61.8675) (end 146.92 62.7062) (width 0.2) (layer "B.Cu") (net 4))
 (segment (start 128.27 52.5462) (end 131.68 52.5462) (width 0.2) (layer "F.Cu") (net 5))
 (segment (start 123.825 56.9912) (end 128.27 52.5462) (width 0.2) (layer "F.Cu") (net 5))
 (segment (start 130.845 52.5462) (end 131.68 52.5462) (width 0.2) (layer "B.Cu") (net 5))
 (segment (start 146.92 65.2462) (end 147.755 65.2462) (width 0.2) (layer "B.Cu") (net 16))
 (segment (start 130.845 57.6262) (end 131.68 57.6262) (width 0.2) (layer "B.Cu") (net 17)))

